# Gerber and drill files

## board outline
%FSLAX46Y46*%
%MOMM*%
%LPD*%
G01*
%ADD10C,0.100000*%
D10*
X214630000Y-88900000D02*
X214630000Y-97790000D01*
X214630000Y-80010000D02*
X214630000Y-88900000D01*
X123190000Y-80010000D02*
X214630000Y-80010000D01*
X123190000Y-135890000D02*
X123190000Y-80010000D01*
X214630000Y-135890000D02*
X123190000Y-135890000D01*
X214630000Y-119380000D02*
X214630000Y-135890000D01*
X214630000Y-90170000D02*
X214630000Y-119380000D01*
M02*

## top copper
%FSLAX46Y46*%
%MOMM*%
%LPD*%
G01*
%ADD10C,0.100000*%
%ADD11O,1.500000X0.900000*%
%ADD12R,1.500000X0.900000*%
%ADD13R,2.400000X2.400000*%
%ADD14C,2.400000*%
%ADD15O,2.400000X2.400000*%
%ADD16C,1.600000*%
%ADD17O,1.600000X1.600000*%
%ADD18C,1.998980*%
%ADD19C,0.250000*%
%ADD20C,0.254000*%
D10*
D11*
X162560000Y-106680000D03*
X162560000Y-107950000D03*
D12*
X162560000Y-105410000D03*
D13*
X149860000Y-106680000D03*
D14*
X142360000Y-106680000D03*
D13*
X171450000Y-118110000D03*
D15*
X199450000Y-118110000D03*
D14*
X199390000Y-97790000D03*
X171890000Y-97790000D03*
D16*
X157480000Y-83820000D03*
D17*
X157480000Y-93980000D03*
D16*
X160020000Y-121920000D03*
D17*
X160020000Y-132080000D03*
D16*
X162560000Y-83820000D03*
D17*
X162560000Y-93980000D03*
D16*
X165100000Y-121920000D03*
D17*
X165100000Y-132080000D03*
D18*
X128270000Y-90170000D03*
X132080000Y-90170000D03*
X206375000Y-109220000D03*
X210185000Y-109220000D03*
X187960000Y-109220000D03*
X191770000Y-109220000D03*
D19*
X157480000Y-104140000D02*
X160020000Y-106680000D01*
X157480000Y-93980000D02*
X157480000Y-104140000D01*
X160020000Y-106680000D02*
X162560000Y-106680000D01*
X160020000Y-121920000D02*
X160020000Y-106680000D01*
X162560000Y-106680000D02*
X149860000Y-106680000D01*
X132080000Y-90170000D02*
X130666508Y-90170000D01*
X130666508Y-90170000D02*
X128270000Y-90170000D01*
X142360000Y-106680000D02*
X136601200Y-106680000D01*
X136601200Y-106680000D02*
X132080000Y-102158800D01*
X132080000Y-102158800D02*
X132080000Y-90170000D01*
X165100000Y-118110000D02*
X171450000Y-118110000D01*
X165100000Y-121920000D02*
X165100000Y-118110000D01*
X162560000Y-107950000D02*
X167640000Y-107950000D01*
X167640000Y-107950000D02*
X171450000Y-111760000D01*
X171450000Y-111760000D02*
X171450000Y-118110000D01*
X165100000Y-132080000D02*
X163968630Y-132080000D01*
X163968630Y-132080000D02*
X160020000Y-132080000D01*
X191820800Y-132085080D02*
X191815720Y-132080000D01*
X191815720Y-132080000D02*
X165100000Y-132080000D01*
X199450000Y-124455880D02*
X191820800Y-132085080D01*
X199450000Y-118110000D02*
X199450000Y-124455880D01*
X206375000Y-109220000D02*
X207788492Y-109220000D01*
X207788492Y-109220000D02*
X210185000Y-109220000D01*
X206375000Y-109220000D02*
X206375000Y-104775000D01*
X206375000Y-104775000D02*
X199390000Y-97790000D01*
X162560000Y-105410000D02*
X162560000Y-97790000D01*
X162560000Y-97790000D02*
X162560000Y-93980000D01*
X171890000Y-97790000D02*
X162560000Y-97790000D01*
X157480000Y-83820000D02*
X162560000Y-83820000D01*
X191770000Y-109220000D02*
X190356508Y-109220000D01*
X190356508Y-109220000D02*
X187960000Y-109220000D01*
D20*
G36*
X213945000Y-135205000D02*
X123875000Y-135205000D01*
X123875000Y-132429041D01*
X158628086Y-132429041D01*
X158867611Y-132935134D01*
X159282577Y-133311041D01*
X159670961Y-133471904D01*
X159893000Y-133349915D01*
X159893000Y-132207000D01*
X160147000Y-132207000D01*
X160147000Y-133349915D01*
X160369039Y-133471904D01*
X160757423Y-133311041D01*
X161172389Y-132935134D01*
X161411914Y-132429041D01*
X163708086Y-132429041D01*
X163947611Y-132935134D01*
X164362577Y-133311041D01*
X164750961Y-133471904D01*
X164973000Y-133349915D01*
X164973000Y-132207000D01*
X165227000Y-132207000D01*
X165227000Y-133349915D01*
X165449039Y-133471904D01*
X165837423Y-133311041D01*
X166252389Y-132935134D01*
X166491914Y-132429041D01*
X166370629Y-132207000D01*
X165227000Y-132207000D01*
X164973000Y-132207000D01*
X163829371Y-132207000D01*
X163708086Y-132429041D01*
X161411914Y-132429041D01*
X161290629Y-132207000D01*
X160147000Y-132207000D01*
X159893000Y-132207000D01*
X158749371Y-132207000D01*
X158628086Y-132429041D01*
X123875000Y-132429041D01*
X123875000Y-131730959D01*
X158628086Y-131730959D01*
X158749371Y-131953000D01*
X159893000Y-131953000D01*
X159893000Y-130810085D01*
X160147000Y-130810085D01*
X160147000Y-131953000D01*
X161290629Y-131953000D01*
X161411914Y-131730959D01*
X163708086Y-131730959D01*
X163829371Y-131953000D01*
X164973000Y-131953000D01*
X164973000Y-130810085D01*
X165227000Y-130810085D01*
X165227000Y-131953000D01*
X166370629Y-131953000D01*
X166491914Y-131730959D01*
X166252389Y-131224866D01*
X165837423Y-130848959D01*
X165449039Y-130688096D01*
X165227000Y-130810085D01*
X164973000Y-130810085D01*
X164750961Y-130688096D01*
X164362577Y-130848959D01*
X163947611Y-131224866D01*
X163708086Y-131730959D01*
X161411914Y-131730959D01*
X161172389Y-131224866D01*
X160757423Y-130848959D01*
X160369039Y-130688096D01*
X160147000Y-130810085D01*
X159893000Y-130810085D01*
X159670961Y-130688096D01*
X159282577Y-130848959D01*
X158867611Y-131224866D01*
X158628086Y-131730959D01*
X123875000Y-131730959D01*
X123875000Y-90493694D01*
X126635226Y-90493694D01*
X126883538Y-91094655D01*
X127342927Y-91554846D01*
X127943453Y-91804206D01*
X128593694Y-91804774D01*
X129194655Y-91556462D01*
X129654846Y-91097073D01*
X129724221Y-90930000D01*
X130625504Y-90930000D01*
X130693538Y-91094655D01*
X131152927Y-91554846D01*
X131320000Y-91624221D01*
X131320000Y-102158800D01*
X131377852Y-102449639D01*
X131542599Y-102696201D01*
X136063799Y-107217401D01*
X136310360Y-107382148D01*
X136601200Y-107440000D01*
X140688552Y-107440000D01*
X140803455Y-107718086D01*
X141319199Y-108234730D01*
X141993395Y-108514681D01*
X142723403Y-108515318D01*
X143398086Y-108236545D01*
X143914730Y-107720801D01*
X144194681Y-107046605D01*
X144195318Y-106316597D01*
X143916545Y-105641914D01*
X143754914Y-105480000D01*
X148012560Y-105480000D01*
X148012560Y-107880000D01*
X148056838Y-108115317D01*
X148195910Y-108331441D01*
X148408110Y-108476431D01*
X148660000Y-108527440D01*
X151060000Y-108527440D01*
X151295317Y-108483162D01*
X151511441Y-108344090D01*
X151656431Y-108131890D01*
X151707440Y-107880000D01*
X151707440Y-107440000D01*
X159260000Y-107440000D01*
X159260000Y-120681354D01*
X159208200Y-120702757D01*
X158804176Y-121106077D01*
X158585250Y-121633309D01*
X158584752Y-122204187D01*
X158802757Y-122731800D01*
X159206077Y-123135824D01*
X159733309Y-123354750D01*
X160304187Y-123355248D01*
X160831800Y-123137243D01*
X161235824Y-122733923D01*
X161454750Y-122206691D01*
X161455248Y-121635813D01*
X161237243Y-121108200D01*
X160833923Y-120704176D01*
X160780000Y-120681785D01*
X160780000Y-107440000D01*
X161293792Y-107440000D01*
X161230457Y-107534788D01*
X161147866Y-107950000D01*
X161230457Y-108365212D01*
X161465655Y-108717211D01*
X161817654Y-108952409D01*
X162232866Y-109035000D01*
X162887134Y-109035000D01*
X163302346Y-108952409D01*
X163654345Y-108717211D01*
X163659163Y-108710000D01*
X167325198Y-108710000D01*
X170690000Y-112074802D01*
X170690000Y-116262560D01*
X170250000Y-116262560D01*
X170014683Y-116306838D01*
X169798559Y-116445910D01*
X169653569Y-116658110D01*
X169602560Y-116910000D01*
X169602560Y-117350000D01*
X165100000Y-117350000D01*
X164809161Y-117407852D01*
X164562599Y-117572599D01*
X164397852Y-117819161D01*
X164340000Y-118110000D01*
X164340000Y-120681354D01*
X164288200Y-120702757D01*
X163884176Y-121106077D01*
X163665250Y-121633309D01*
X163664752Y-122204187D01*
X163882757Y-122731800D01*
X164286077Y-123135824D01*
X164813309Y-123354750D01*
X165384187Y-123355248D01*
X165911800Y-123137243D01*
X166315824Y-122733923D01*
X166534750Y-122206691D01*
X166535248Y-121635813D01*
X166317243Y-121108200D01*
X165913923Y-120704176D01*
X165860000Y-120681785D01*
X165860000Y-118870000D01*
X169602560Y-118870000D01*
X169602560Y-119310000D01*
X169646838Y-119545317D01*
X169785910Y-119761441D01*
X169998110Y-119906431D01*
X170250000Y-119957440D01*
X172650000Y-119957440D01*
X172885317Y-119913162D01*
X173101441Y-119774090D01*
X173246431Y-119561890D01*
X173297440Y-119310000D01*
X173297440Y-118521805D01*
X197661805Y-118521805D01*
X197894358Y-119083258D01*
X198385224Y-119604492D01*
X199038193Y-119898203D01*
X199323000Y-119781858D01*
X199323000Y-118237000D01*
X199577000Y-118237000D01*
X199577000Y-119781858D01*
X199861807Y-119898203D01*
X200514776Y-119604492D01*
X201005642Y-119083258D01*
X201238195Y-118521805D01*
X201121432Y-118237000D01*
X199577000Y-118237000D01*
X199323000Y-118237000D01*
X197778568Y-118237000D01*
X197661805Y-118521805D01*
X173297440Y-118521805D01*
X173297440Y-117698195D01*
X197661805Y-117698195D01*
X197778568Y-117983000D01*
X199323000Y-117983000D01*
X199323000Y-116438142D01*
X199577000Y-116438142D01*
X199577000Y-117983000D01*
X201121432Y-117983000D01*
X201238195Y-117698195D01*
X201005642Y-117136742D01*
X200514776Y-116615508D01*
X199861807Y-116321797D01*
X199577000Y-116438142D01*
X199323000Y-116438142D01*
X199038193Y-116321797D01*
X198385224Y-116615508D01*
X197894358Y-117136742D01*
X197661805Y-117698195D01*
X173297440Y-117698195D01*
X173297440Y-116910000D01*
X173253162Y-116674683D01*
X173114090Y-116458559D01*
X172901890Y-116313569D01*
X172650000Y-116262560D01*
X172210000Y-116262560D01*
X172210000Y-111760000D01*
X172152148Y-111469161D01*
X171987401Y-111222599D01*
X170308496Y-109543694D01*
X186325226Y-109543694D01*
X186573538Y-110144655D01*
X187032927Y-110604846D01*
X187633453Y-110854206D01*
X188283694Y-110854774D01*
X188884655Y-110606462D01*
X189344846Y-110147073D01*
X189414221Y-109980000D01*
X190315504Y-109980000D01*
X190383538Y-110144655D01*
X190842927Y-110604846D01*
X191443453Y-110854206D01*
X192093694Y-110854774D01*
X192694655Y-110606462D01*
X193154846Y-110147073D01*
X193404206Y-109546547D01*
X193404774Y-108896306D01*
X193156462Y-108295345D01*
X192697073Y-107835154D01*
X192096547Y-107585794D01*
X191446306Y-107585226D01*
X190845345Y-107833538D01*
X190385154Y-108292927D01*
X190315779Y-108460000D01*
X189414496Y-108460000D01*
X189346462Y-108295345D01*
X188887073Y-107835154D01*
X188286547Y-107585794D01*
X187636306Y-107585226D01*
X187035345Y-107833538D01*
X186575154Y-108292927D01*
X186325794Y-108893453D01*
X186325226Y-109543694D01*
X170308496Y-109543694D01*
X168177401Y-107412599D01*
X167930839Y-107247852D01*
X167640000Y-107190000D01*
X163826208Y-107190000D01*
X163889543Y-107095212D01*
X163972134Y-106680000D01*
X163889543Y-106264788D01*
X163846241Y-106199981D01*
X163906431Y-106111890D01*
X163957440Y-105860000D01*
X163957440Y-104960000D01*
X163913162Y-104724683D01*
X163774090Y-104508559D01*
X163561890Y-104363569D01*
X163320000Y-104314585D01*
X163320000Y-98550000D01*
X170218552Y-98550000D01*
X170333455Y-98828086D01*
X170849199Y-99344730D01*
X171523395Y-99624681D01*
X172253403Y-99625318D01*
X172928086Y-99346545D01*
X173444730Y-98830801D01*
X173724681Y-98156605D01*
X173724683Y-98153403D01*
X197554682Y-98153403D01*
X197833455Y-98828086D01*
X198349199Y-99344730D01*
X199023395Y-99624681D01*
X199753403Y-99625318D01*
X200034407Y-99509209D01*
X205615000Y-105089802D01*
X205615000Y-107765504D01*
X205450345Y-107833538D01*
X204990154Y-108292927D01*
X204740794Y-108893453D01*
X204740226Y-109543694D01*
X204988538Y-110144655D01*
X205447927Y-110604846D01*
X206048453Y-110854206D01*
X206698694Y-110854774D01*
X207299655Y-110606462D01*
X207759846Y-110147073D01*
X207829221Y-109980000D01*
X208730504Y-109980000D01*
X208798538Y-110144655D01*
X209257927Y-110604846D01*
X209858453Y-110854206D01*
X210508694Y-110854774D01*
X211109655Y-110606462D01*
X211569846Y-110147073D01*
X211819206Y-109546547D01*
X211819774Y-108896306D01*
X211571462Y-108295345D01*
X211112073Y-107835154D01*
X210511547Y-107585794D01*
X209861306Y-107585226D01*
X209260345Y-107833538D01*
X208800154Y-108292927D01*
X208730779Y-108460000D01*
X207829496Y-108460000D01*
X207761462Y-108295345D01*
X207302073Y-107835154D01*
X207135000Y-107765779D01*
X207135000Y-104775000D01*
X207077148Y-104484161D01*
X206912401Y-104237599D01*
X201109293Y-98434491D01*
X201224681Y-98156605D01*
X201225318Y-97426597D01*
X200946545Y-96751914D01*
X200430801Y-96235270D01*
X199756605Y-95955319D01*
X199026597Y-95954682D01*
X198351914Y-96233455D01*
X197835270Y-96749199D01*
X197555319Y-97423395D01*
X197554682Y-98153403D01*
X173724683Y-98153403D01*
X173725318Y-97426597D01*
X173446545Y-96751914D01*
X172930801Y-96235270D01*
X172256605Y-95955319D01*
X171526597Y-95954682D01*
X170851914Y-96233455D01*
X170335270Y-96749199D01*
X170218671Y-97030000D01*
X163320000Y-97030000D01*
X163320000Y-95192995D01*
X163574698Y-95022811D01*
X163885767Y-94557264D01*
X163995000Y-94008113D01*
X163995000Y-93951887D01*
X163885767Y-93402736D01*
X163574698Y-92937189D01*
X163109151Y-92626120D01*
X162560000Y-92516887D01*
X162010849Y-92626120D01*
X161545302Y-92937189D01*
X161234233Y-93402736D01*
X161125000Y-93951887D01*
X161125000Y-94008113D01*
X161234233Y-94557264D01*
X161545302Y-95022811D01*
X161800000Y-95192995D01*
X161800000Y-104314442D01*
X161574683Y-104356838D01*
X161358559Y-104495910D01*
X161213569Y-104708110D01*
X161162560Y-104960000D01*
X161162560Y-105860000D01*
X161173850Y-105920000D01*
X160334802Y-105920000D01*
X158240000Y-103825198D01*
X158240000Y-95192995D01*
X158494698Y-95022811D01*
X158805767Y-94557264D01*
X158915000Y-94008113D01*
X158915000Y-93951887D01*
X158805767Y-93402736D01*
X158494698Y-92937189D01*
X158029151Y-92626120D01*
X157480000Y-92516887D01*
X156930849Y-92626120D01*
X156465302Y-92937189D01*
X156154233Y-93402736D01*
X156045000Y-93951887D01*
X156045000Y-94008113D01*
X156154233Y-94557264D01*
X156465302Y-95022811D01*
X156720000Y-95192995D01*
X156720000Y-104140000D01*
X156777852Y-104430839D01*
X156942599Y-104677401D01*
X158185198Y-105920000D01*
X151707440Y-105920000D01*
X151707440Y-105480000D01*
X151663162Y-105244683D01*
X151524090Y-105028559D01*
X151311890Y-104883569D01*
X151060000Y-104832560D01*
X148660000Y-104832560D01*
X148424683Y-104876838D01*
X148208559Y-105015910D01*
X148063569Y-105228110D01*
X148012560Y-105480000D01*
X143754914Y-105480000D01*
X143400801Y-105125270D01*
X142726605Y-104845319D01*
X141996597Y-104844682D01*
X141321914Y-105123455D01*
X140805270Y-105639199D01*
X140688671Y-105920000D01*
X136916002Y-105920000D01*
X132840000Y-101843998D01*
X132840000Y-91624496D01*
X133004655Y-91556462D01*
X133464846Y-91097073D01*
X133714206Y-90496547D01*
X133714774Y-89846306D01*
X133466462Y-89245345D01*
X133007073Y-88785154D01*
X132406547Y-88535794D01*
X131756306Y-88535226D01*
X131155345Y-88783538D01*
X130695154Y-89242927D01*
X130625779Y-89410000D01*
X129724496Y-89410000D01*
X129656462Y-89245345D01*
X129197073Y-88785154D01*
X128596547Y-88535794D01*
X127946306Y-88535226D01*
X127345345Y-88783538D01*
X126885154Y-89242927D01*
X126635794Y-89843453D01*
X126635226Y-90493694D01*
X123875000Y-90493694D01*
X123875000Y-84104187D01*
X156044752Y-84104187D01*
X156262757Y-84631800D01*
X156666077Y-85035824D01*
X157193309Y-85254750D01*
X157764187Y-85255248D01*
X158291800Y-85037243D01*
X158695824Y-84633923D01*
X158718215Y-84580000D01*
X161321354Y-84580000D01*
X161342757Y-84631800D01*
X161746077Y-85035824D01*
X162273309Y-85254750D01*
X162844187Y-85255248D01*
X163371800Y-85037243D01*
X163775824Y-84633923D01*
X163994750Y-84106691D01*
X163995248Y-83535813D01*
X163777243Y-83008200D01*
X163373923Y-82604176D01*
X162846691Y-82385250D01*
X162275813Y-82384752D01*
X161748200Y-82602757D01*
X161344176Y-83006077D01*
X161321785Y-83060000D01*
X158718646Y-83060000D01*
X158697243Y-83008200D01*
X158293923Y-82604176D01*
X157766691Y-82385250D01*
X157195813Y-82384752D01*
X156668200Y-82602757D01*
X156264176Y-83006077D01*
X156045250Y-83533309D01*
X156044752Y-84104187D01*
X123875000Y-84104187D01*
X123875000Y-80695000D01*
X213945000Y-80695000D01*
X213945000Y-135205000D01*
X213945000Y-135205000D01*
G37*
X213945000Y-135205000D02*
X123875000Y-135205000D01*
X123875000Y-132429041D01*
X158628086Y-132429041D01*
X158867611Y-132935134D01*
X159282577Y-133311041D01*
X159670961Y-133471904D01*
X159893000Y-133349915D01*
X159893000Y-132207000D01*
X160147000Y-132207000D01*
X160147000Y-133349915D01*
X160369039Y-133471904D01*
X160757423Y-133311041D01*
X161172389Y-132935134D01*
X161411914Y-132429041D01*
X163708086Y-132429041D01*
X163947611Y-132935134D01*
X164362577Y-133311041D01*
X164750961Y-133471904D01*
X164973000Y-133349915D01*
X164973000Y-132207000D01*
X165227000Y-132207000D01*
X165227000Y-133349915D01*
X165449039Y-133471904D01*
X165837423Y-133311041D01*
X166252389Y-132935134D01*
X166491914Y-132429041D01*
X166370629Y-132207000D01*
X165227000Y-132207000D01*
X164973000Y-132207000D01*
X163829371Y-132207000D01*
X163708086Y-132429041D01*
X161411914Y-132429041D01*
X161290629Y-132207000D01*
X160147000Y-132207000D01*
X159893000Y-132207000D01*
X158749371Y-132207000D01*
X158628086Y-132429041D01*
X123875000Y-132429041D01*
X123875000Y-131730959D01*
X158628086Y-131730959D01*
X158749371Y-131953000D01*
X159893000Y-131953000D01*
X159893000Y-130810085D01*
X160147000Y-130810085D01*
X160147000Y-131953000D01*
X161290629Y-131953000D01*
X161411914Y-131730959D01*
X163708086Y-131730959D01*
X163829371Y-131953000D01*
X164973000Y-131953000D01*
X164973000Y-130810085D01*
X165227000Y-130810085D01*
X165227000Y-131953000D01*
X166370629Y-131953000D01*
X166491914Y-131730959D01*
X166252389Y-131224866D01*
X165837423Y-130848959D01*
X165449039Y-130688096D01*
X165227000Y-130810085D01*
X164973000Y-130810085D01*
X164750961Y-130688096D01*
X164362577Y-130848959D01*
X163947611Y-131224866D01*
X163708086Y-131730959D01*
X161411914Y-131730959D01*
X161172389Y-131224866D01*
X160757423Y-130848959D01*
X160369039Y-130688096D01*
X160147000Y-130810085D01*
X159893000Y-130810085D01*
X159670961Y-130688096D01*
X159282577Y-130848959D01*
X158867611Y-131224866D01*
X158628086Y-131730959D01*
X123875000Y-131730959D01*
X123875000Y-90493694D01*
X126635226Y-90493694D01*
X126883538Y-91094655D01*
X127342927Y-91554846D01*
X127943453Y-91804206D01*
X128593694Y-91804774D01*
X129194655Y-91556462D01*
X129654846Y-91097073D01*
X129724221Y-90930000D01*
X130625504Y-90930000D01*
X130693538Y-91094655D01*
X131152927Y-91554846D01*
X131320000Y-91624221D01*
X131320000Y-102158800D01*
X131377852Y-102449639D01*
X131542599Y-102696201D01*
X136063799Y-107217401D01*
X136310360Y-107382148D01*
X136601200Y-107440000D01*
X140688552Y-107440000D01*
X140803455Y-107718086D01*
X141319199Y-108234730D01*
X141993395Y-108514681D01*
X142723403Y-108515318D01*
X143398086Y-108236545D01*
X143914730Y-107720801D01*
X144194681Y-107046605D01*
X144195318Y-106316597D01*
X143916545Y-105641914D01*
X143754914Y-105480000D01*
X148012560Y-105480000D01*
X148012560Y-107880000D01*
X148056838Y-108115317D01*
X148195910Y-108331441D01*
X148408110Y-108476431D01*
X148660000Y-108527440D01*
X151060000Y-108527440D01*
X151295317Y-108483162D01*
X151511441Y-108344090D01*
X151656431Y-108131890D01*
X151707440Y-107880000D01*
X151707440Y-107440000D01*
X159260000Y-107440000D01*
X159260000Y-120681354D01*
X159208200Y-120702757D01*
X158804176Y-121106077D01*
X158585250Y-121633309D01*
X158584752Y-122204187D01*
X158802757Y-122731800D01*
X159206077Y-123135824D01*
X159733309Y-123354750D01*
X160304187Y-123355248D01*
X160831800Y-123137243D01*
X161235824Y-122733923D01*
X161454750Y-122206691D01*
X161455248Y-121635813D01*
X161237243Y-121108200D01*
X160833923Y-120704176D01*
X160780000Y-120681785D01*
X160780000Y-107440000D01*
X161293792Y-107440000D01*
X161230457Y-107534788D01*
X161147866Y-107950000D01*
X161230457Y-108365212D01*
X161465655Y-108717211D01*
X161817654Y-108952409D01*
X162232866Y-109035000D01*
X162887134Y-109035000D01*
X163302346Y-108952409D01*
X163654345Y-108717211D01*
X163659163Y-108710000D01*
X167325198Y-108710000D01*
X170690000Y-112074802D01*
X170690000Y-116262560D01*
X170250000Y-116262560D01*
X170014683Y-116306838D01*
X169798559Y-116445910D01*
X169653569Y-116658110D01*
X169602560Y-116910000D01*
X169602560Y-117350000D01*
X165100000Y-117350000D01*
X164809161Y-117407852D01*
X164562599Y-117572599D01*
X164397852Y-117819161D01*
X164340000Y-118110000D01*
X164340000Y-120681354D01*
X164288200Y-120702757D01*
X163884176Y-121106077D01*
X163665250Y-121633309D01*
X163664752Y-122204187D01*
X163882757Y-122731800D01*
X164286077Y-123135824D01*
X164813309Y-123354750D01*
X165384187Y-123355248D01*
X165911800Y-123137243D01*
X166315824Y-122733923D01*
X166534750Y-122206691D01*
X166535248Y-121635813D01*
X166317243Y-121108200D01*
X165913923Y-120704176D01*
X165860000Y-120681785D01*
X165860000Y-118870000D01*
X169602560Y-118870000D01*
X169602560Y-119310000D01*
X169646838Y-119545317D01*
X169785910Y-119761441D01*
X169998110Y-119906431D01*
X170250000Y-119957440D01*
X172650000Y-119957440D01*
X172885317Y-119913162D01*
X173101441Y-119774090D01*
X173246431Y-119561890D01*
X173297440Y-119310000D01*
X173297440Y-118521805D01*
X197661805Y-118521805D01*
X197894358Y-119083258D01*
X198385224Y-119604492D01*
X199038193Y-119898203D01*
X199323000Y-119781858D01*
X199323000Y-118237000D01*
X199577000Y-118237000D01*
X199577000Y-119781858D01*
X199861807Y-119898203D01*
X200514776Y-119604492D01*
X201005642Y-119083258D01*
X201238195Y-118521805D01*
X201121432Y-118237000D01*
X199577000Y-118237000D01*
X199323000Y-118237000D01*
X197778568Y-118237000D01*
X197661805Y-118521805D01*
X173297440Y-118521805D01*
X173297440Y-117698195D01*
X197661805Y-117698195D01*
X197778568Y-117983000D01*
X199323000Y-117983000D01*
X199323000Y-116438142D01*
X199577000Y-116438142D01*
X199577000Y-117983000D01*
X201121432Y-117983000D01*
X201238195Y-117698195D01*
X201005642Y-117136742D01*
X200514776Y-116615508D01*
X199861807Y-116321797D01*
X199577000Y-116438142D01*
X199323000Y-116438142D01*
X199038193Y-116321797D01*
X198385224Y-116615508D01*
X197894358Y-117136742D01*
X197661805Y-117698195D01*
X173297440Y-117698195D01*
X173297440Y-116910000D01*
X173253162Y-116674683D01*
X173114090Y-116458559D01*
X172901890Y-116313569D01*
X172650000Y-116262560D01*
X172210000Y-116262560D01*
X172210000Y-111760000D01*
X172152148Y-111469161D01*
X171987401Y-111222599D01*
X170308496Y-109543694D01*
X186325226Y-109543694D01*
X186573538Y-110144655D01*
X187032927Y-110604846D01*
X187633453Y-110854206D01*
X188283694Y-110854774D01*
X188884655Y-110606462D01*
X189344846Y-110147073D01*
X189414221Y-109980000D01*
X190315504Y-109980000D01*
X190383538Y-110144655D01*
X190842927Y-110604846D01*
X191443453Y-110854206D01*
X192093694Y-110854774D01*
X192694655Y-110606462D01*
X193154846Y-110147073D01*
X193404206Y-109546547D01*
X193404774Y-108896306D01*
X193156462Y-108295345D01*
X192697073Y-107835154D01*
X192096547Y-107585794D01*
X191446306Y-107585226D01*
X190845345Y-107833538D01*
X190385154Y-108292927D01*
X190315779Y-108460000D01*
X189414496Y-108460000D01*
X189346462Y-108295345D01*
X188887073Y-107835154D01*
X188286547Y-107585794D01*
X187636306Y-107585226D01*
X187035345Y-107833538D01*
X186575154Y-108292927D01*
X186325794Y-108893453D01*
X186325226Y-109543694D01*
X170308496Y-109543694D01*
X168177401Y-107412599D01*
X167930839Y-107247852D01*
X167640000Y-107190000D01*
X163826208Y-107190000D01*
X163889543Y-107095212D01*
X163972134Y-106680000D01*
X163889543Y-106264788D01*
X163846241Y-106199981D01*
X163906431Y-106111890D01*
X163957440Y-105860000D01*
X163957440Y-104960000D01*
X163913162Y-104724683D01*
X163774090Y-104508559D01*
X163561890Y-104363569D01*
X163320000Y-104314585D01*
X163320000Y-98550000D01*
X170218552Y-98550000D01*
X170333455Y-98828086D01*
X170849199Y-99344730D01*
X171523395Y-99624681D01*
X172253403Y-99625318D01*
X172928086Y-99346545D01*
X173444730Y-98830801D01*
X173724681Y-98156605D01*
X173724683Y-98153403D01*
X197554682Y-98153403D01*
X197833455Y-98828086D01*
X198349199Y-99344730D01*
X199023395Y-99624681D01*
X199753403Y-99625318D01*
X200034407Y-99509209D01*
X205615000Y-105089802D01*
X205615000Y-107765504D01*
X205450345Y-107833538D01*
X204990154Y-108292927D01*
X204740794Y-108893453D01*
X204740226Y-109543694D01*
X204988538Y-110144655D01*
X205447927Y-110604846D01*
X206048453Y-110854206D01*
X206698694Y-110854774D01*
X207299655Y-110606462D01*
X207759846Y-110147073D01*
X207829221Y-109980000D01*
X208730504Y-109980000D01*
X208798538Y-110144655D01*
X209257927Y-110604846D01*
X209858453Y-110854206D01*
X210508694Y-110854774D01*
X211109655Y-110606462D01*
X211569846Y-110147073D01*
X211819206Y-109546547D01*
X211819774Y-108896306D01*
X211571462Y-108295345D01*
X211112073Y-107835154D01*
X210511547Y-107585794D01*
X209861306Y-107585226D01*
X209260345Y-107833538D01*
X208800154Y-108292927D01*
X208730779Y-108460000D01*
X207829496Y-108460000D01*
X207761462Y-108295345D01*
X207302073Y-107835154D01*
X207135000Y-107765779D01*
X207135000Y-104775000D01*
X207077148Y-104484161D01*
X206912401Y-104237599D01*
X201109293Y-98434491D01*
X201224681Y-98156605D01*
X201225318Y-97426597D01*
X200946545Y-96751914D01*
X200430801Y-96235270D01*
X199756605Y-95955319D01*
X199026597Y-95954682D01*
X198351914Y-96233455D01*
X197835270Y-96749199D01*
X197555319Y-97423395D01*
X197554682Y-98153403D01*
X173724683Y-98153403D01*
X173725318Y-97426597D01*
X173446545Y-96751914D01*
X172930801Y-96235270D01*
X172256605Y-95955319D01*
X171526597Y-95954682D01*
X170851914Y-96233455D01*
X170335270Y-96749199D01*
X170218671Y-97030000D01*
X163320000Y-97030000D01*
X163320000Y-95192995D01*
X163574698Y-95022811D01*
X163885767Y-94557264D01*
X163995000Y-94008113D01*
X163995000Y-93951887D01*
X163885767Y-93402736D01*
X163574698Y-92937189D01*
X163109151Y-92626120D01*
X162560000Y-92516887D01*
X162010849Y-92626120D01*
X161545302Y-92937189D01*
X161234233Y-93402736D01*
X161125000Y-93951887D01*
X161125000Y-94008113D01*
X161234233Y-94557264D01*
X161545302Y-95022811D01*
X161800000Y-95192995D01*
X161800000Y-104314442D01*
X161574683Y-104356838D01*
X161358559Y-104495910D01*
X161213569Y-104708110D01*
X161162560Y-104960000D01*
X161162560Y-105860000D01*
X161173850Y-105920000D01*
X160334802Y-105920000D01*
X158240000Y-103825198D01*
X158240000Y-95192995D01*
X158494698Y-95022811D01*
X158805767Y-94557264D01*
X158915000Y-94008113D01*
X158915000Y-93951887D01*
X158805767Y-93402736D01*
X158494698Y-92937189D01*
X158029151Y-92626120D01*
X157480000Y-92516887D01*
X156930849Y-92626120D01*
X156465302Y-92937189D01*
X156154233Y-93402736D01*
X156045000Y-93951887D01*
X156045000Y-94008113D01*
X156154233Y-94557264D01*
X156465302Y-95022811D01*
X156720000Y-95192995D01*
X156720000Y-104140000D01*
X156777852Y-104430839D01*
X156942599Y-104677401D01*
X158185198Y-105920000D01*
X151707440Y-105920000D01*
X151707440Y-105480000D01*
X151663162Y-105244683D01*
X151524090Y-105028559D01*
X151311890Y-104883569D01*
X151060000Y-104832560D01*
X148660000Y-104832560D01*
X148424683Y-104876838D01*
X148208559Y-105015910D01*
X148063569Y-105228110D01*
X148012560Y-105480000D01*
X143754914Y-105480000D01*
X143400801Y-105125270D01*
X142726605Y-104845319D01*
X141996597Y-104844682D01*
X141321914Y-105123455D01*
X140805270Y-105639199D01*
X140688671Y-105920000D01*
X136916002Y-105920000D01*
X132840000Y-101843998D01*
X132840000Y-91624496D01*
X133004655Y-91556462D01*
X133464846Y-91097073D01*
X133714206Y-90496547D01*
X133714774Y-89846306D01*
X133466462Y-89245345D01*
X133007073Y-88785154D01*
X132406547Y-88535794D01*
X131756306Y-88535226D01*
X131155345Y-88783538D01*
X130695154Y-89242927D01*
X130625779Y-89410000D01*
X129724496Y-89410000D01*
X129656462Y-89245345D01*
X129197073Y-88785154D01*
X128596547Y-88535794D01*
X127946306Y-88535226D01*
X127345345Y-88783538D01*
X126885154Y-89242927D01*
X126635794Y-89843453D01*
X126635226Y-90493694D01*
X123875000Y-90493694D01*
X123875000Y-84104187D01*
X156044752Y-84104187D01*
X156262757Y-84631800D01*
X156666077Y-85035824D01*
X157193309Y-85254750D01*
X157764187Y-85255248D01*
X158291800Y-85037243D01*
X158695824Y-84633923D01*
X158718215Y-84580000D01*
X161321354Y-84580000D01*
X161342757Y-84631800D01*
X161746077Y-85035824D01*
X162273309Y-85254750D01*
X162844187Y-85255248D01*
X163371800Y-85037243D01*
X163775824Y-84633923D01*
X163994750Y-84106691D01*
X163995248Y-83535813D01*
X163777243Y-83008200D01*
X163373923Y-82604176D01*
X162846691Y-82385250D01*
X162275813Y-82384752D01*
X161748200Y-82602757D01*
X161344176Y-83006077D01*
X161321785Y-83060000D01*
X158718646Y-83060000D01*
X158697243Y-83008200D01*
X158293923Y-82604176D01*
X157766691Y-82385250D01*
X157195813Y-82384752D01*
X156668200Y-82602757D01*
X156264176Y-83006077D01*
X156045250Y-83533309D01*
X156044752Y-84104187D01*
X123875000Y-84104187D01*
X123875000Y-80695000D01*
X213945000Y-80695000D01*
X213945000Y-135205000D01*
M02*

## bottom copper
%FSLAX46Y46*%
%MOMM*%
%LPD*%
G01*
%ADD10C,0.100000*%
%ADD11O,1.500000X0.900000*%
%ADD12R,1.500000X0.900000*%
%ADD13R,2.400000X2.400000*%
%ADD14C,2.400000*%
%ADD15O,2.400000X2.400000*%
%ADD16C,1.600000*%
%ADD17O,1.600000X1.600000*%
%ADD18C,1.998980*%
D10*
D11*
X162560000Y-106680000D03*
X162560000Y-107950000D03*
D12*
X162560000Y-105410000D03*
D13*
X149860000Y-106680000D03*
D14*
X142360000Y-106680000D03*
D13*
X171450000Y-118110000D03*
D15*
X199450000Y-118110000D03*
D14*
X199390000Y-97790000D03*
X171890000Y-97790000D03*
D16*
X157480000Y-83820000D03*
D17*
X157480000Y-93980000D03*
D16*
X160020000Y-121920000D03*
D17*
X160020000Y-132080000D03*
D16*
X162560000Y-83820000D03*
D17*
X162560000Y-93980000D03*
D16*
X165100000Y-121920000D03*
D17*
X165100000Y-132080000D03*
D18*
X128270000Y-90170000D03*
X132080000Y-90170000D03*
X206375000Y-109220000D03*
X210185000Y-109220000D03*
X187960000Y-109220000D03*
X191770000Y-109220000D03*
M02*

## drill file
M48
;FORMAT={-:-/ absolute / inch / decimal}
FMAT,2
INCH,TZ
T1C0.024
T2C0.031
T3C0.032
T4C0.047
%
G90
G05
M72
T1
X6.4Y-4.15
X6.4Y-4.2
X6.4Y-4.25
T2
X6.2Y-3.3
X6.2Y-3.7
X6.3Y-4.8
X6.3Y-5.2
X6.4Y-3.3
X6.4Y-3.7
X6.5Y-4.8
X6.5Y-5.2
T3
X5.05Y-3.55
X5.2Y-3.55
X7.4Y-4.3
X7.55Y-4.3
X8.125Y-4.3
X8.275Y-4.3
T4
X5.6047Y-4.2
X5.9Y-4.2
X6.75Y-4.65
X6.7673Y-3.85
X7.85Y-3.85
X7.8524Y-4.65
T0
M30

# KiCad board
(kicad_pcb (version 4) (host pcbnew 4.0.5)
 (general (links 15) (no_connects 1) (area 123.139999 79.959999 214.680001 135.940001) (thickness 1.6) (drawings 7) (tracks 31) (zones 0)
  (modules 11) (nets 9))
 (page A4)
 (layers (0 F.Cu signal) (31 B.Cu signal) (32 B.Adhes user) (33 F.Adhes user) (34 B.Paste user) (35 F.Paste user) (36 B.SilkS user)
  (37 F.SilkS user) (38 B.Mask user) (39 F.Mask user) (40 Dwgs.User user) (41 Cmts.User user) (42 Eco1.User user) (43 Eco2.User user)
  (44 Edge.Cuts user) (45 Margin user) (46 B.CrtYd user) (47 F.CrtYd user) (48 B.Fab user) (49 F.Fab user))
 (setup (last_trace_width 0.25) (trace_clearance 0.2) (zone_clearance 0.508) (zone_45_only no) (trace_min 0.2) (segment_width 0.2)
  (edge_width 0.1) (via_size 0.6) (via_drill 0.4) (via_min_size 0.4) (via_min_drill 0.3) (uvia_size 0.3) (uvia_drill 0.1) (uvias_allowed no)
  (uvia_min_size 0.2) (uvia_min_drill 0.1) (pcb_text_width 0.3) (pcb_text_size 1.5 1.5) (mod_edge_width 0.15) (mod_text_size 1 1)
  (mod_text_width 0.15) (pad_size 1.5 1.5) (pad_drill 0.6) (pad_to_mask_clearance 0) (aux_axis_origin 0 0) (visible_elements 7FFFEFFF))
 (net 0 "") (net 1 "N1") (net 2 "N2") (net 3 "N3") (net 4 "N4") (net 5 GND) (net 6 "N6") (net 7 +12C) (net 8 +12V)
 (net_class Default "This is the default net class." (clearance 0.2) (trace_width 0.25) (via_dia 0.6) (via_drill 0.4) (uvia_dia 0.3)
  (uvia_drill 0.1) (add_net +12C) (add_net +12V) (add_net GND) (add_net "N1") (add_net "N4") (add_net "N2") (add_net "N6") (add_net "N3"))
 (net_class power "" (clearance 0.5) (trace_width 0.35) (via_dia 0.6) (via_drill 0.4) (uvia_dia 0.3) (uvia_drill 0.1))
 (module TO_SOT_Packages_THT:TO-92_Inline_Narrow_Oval (layer F.Cu) (at 162.56 105.41 270)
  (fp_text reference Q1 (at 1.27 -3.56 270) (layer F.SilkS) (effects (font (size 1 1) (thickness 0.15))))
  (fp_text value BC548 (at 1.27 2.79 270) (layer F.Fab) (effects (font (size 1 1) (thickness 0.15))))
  (pad 2 thru_hole oval (at 1.27 0 90) (size 0.9 1.5) (drill 0.6) (layers *.Cu *.Mask) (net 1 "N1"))
  (pad 3 thru_hole oval (at 2.54 0 90) (size 0.9 1.5) (drill 0.6) (layers *.Cu *.Mask) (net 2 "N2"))
  (pad 1 thru_hole rect (at 0 0 90) (size 0.9 1.5) (drill 0.6) (layers *.Cu *.Mask) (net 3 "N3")))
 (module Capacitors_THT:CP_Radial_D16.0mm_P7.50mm (layer F.Cu) (at 149.86 106.68 180)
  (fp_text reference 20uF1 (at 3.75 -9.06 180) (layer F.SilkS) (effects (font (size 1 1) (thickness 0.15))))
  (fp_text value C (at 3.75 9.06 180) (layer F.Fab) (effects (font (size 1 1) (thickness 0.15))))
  (pad 1 thru_hole rect (at 0 0 180) (size 2.4 2.4) (drill 1.2) (layers *.Cu *.Mask) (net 1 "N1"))
  (pad 2 thru_hole circle (at 7.5 0 180) (size 2.4 2.4) (drill 1.2) (layers *.Cu *.Mask) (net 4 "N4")))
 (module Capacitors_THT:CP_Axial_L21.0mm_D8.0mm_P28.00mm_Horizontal (layer F.Cu) (at 171.45 118.11)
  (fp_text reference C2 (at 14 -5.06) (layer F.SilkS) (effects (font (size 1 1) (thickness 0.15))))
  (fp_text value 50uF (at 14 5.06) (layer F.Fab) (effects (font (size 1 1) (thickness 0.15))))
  (pad 1 thru_hole rect (at 0 0) (size 2.4 2.4) (drill 1.2) (layers *.Cu *.Mask) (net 2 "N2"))
  (pad 2 thru_hole oval (at 28 0) (size 2.4 2.4) (drill 1.2) (layers *.Cu *.Mask) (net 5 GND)))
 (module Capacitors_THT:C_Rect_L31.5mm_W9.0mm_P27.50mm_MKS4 (layer F.Cu) (at 199.39 97.79 180)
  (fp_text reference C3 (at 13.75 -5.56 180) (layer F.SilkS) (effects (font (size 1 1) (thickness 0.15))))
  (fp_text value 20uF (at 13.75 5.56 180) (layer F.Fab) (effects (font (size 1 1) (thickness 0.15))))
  (pad 1 thru_hole circle (at 0 0 180) (size 2.4 2.4) (drill 1.2) (layers *.Cu *.Mask) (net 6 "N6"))
  (pad 2 thru_hole circle (at 27.5 0 180) (size 2.4 2.4) (drill 1.2) (layers *.Cu *.Mask) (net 3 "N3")))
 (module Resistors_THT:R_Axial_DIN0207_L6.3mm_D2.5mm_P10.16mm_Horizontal (layer F.Cu) (at 157.48 83.82 270)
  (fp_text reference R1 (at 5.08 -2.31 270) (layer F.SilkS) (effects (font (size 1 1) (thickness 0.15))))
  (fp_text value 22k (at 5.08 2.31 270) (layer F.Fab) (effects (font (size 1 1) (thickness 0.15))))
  (pad 1 thru_hole circle (at 0 0 270) (size 1.6 1.6) (drill 0.8) (layers *.Cu *.Mask) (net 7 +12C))
  (pad 2 thru_hole oval (at 10.16 0 270) (size 1.6 1.6) (drill 0.8) (layers *.Cu *.Mask) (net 1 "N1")))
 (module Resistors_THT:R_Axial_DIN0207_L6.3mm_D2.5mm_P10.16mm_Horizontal (layer F.Cu) (at 160.02 121.92 270)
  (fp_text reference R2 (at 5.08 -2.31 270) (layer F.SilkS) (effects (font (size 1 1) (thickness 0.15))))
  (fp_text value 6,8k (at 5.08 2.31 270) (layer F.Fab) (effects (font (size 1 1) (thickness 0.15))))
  (pad 1 thru_hole circle (at 0 0 270) (size 1.6 1.6) (drill 0.8) (layers *.Cu *.Mask) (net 1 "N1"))
  (pad 2 thru_hole oval (at 10.16 0 270) (size 1.6 1.6) (drill 0.8) (layers *.Cu *.Mask) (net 5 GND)))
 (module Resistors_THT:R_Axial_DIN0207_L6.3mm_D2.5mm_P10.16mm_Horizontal (layer F.Cu) (at 162.56 83.82 270)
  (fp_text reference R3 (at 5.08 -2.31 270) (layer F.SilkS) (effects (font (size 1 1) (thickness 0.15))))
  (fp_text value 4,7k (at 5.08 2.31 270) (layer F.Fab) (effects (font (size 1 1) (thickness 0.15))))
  (pad 1 thru_hole circle (at 0 0 270) (size 1.6 1.6) (drill 0.8) (layers *.Cu *.Mask) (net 7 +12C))
  (pad 2 thru_hole oval (at 10.16 0 270) (size 1.6 1.6) (drill 0.8) (layers *.Cu *.Mask) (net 3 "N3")))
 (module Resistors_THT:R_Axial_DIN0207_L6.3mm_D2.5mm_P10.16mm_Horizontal (layer F.Cu) (at 165.1 121.92 270)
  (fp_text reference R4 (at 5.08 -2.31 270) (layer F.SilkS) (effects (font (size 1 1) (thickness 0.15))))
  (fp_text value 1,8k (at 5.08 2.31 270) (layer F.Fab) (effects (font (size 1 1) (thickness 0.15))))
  (pad 1 thru_hole circle (at 0 0 270) (size 1.6 1.6) (drill 0.8) (layers *.Cu *.Mask) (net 2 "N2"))
  (pad 2 thru_hole oval (at 10.16 0 270) (size 1.6 1.6) (drill 0.8) (layers *.Cu *.Mask) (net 5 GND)))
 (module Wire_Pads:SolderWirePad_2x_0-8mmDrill (layer F.Cu) (at 130.175 90.17)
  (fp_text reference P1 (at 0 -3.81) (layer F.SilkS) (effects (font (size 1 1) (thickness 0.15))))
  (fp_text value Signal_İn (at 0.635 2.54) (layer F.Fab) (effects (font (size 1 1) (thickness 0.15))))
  (pad 1 thru_hole circle (at -1.905 0) (size 1.99898 1.99898) (drill 0.8001) (layers *.Cu *.Mask) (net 4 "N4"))
  (pad 1 thru_hole circle (at 1.905 0) (size 1.99898 1.99898) (drill 0.8001) (layers *.Cu *.Mask) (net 4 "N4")))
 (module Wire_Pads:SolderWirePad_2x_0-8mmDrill (layer F.Cu) (at 208.28 109.22)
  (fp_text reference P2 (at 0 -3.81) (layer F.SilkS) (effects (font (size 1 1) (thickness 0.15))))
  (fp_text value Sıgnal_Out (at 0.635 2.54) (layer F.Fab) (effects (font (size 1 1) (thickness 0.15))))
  (pad 1 thru_hole circle (at -1.905 0) (size 1.99898 1.99898) (drill 0.8001) (layers *.Cu *.Mask) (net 6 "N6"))
  (pad 1 thru_hole circle (at 1.905 0) (size 1.99898 1.99898) (drill 0.8001) (layers *.Cu *.Mask) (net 6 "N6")))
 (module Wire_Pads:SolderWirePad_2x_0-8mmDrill (layer F.Cu) (at 189.865 109.22)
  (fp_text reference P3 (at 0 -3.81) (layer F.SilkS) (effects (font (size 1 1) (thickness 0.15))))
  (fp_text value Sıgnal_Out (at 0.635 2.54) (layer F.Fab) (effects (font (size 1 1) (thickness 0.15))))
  (pad 1 thru_hole circle (at -1.905 0) (size 1.99898 1.99898) (drill 0.8001) (layers *.Cu *.Mask) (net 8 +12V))
  (pad 1 thru_hole circle (at 1.905 0) (size 1.99898 1.99898) (drill 0.8001) (layers *.Cu *.Mask) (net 8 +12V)))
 (gr_line (start 214.63 88.9) (end 214.63 97.79) (layer Edge.Cuts) (width 0.1))
 (gr_line (start 214.63 80.01) (end 214.63 88.9) (layer Edge.Cuts) (width 0.1))
 (gr_line (start 123.19 80.01) (end 214.63 80.01) (layer Edge.Cuts) (width 0.1))
 (gr_line (start 123.19 135.89) (end 123.19 80.01) (layer Edge.Cuts) (width 0.1))
 (gr_line (start 214.63 135.89) (end 123.19 135.89) (layer Edge.Cuts) (width 0.1))
 (gr_line (start 214.63 119.38) (end 214.63 135.89) (layer Edge.Cuts) (width 0.1))
 (gr_line (start 214.63 90.17) (end 214.63 119.38) (layer Edge.Cuts) (width 0.1))
 (segment (start 157.48 104.14) (end 160.02 106.68) (width 0.25) (layer F.Cu) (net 1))
 (segment (start 157.48 93.98) (end 157.48 104.14) (width 0.25) (layer F.Cu) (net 1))
 (segment (start 160.02 106.68) (end 162.56 106.68) (width 0.25) (layer F.Cu) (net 1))
 (segment (start 160.02 121.92) (end 160.02 106.68) (width 0.25) (layer F.Cu) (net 1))
 (segment (start 162.56 106.68) (end 149.86 106.68) (width 0.25) (layer F.Cu) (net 1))
 (segment (start 132.08 90.17) (end 130.666508 90.17) (width 0.25) (layer F.Cu) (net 4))
 (segment (start 130.666508 90.17) (end 128.27 90.17) (width 0.25) (layer F.Cu) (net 4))
 (segment (start 142.36 106.68) (end 136.6012 106.68) (width 0.25) (layer F.Cu) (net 4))
 (segment (start 136.6012 106.68) (end 132.08 102.1588) (width 0.25) (layer F.Cu) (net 4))
 (segment (start 132.08 102.1588) (end 132.08 90.17) (width 0.25) (layer F.Cu) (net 4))
 (segment (start 165.1 118.11) (end 171.45 118.11) (width 0.25) (layer F.Cu) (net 2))
 (segment (start 165.1 121.92) (end 165.1 118.11) (width 0.25) (layer F.Cu) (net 2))
 (segment (start 162.56 107.95) (end 167.64 107.95) (width 0.25) (layer F.Cu) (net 2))
 (segment (start 167.64 107.95) (end 171.45 111.76) (width 0.25) (layer F.Cu) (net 2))
 (segment (start 171.45 111.76) (end 171.45 118.11) (width 0.25) (layer F.Cu) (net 2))
 (segment (start 165.1 132.08) (end 163.96863 132.08) (width 0.25) (layer F.Cu) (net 5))
 (segment (start 163.96863 132.08) (end 160.02 132.08) (width 0.25) (layer F.Cu) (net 5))
 (segment (start 191.8208 132.08508) (end 191.81572 132.08) (width 0.25) (layer F.Cu) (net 5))
 (segment (start 191.81572 132.08) (end 165.1 132.08) (width 0.25) (layer F.Cu) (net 5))
 (segment (start 199.45 124.45588) (end 191.8208 132.08508) (width 0.25) (layer F.Cu) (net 5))
 (segment (start 199.45 118.11) (end 199.45 124.45588) (width 0.25) (layer F.Cu) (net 5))
 (segment (start 206.375 109.22) (end 207.788492 109.22) (width 0.25) (layer F.Cu) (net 6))
 (segment (start 207.788492 109.22) (end 210.185 109.22) (width 0.25) (layer F.Cu) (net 6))
 (segment (start 206.375 109.22) (end 206.375 104.775) (width 0.25) (layer F.Cu) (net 6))
 (segment (start 206.375 104.775) (end 199.39 97.79) (width 0.25) (layer F.Cu) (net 6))
 (segment (start 162.56 105.41) (end 162.56 97.79) (width 0.25) (layer F.Cu) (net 3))
 (segment (start 162.56 97.79) (end 162.56 93.98) (width 0.25) (layer F.Cu) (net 3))
 (segment (start 171.89 97.79) (end 162.56 97.79) (width 0.25) (layer F.Cu) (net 3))
 (segment (start 157.48 83.82) (end 162.56 83.82) (width 0.25) (layer F.Cu) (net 7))
 (segment (start 191.77 109.22) (end 190.356508 109.22) (width 0.25) (layer F.Cu) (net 8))
 (segment (start 190.356508 109.22) (end 187.96 109.22) (width 0.25) (layer F.Cu) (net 8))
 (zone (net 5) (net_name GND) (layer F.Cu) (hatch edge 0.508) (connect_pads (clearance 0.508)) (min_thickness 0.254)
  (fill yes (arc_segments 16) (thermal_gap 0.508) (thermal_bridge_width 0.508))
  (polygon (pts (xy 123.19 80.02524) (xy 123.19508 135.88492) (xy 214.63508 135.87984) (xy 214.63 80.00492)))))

